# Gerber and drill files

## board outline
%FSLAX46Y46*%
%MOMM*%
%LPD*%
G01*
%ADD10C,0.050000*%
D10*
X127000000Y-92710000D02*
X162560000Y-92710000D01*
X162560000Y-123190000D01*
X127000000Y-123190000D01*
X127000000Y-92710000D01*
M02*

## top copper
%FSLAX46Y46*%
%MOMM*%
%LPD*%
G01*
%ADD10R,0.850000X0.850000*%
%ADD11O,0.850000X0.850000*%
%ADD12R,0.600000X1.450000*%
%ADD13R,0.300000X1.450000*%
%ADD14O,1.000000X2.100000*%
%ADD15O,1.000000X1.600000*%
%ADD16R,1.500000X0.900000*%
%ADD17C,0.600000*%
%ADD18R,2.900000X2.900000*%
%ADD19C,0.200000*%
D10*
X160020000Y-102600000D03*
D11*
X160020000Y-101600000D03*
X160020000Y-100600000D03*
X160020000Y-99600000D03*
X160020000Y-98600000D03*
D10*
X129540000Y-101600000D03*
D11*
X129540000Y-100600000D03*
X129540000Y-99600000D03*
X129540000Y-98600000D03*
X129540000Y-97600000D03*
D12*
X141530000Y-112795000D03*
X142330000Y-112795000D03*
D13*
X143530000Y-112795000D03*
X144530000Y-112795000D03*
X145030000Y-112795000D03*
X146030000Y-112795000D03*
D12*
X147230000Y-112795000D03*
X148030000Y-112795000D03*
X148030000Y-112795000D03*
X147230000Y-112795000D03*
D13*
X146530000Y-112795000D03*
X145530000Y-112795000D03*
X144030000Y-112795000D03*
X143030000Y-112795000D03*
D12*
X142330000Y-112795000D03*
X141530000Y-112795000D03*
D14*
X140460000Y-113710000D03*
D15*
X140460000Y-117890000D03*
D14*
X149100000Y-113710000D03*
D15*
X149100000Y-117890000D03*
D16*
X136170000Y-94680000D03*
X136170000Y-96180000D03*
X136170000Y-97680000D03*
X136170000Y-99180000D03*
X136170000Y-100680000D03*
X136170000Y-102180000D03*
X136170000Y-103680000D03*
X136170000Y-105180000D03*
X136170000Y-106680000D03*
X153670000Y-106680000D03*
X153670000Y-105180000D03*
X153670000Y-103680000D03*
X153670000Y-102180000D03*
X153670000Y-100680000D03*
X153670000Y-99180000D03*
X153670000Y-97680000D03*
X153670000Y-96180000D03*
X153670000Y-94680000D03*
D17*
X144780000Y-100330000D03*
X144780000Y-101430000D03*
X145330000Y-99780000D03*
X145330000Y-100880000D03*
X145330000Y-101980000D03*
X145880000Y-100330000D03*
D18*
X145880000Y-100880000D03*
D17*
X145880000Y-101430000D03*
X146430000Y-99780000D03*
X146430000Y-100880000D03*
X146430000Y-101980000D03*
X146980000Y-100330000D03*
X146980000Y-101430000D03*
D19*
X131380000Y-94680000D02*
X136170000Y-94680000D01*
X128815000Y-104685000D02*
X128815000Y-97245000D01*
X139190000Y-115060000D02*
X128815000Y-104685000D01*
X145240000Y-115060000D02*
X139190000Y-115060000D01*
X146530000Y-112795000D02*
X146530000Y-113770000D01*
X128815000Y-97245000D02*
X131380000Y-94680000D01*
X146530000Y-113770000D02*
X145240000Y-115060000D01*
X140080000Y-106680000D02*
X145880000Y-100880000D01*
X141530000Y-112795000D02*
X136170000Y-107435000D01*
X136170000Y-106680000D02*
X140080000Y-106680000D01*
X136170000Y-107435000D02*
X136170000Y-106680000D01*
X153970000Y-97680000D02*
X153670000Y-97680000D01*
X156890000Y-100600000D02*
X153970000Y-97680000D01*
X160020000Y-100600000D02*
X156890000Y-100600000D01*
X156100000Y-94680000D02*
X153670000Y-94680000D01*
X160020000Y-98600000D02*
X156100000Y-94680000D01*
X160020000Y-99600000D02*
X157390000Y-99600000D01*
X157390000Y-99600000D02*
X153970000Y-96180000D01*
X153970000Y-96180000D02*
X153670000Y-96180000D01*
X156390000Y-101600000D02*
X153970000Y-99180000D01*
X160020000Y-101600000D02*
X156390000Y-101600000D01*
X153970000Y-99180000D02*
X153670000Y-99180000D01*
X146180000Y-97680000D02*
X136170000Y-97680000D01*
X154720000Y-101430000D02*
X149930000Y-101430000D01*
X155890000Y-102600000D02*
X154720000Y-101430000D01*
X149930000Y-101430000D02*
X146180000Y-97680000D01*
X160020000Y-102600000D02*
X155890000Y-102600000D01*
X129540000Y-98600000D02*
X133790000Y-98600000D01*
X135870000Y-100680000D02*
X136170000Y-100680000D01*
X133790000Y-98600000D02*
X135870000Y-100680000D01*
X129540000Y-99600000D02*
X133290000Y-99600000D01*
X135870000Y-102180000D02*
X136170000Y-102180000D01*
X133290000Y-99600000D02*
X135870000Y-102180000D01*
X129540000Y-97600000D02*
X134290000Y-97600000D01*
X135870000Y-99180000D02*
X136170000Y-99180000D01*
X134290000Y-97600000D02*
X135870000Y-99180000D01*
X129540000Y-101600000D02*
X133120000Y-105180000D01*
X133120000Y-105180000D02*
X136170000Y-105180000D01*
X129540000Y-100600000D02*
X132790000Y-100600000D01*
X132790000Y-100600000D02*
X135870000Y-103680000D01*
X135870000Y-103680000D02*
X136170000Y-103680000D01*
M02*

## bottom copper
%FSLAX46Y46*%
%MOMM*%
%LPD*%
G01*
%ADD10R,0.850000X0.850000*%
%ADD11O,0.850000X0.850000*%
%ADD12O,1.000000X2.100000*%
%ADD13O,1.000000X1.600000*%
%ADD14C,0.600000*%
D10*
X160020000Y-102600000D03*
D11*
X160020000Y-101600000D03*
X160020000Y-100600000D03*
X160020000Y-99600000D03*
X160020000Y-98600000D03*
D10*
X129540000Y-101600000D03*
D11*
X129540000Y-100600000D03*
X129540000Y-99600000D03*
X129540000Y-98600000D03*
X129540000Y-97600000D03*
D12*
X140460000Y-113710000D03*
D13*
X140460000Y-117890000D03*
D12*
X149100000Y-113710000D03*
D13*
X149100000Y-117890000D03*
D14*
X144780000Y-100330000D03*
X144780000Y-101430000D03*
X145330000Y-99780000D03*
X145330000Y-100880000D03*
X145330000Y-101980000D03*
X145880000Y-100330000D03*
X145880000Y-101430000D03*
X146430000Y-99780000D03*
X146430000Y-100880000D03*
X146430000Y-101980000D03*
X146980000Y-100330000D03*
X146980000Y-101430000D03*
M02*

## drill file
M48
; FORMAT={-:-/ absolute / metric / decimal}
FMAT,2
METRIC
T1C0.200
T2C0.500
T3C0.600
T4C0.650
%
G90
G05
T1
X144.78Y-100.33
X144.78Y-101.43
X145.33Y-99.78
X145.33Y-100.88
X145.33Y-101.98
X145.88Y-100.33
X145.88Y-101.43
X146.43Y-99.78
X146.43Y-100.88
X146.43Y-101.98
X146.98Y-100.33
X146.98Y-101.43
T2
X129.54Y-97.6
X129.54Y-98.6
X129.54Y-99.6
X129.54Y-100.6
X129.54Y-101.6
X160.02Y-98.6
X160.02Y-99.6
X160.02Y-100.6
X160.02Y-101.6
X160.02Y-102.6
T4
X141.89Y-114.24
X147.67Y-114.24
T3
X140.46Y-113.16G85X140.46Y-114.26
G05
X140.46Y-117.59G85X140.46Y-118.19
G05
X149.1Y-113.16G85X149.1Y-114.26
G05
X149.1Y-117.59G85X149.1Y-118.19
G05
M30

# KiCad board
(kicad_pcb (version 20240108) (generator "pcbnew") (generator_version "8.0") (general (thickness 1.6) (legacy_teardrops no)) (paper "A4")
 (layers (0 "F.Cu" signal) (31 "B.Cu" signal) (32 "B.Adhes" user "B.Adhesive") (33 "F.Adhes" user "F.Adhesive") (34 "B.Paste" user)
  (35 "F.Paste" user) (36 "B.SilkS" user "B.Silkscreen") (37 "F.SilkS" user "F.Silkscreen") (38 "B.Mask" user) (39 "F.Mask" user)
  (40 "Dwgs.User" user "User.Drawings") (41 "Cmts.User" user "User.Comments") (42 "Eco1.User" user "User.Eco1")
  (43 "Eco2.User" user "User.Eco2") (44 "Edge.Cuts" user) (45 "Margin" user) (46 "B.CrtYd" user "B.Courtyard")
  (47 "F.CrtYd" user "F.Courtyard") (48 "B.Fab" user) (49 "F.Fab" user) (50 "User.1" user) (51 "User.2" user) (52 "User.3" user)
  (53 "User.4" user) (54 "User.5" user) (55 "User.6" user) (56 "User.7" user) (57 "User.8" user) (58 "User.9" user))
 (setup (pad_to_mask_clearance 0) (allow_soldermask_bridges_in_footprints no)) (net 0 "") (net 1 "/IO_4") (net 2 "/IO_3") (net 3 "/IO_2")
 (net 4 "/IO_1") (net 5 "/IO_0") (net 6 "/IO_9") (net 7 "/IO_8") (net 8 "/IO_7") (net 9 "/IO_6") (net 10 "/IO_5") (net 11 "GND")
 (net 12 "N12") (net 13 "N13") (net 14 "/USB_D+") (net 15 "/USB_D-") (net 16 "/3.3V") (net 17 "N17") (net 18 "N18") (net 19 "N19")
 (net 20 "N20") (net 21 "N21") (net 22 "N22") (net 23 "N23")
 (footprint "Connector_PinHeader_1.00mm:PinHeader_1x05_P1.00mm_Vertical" (layer "F.Cu") (at 160.02 102.6 180)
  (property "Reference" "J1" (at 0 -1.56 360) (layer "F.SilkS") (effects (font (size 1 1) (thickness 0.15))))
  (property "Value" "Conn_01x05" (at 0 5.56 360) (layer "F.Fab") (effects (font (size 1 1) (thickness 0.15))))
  (pad "1" thru_hole rect (at 0 0 180) (size 0.85 0.85) (drill 0.5) (layers "*.Cu" "*.Mask") (remove_unused_layers no) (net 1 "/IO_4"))
  (pad "2" thru_hole oval (at 0 1 180) (size 0.85 0.85) (drill 0.5) (layers "*.Cu" "*.Mask") (remove_unused_layers no) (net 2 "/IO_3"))
  (pad "3" thru_hole oval (at 0 2 180) (size 0.85 0.85) (drill 0.5) (layers "*.Cu" "*.Mask") (remove_unused_layers no) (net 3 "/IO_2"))
  (pad "4" thru_hole oval (at 0 3 180) (size 0.85 0.85) (drill 0.5) (layers "*.Cu" "*.Mask") (remove_unused_layers no) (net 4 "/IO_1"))
  (pad "5" thru_hole oval (at 0 4 180) (size 0.85 0.85) (drill 0.5) (layers "*.Cu" "*.Mask") (remove_unused_layers no) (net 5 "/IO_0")))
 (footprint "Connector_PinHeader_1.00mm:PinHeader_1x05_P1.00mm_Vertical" (layer "F.Cu") (at 129.54 101.6 180)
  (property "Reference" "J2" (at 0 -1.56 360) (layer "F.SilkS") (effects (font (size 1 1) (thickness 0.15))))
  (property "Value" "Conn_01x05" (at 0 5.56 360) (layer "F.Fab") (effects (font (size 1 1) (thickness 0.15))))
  (pad "1" thru_hole rect (at 0 0 180) (size 0.85 0.85) (drill 0.5) (layers "*.Cu" "*.Mask") (remove_unused_layers no) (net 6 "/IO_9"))
  (pad "2" thru_hole oval (at 0 1 180) (size 0.85 0.85) (drill 0.5) (layers "*.Cu" "*.Mask") (remove_unused_layers no) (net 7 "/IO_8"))
  (pad "3" thru_hole oval (at 0 2 180) (size 0.85 0.85) (drill 0.5) (layers "*.Cu" "*.Mask") (remove_unused_layers no) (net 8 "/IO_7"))
  (pad "4" thru_hole oval (at 0 3 180) (size 0.85 0.85) (drill 0.5) (layers "*.Cu" "*.Mask") (remove_unused_layers no) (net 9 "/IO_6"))
  (pad "5" thru_hole oval (at 0 4 180) (size 0.85 0.85) (drill 0.5) (layers "*.Cu" "*.Mask") (remove_unused_layers no) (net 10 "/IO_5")))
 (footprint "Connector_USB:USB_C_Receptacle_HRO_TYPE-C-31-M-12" (layer "F.Cu") (at 144.78 116.84)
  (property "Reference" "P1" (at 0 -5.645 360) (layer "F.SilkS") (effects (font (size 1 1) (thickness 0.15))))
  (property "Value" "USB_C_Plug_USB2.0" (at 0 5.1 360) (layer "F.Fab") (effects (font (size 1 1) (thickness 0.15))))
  (pad "" np_thru_hole circle (at -2.89 -2.6) (size 0.65 0.65) (drill 0.65) (layers "*.Cu" "*.Mask"))
  (pad "" np_thru_hole circle (at 2.89 -2.6) (size 0.65 0.65) (drill 0.65) (layers "*.Cu" "*.Mask"))
  (pad "A1" smd rect (at -3.25 -4.045) (size 0.6 1.45) (layers "F.Cu" "F.Paste" "F.Mask") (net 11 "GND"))
  (pad "A4" smd rect (at -2.45 -4.045) (size 0.6 1.45) (layers "F.Cu" "F.Paste" "F.Mask") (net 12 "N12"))
  (pad "A5" smd rect (at -1.25 -4.045) (size 0.3 1.45) (layers "F.Cu" "F.Paste" "F.Mask") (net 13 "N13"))
  (pad "A6" smd rect (at -0.25 -4.045) (size 0.3 1.45) (layers "F.Cu" "F.Paste" "F.Mask") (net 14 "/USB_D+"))
  (pad "A7" smd rect (at 0.25 -4.045) (size 0.3 1.45) (layers "F.Cu" "F.Paste" "F.Mask") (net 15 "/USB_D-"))
  (pad "A8" smd rect (at 1.25 -4.045) (size 0.3 1.45) (layers "F.Cu" "F.Paste" "F.Mask"))
  (pad "A9" smd rect (at 2.45 -4.045) (size 0.6 1.45) (layers "F.Cu" "F.Paste" "F.Mask") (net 12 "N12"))
  (pad "A12" smd rect (at 3.25 -4.045) (size 0.6 1.45) (layers "F.Cu" "F.Paste" "F.Mask") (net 11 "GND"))
  (pad "B1" smd rect (at 3.25 -4.045) (size 0.6 1.45) (layers "F.Cu" "F.Paste" "F.Mask") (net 11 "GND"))
  (pad "B4" smd rect (at 2.45 -4.045) (size 0.6 1.45) (layers "F.Cu" "F.Paste" "F.Mask") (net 12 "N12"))
  (pad "B5" smd rect (at 1.75 -4.045) (size 0.3 1.45) (layers "F.Cu" "F.Paste" "F.Mask") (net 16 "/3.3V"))
  (pad "B6" smd rect (at 0.75 -4.045) (size 0.3 1.45) (layers "F.Cu" "F.Paste" "F.Mask"))
  (pad "B7" smd rect (at -0.75 -4.045) (size 0.3 1.45) (layers "F.Cu" "F.Paste" "F.Mask"))
  (pad "B8" smd rect (at -1.75 -4.045) (size 0.3 1.45) (layers "F.Cu" "F.Paste" "F.Mask"))
  (pad "B9" smd rect (at -2.45 -4.045) (size 0.6 1.45) (layers "F.Cu" "F.Paste" "F.Mask") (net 12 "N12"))
  (pad "B12" smd rect (at -3.25 -4.045) (size 0.6 1.45) (layers "F.Cu" "F.Paste" "F.Mask") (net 11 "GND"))
  (pad "S1" thru_hole oval (at -4.32 -3.13) (size 1 2.1) (drill oval 0.6 1.7) (layers "*.Cu" "*.Mask") (remove_unused_layers no)
   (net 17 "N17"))
  (pad "S1" thru_hole oval (at -4.32 1.05) (size 1 1.6) (drill oval 0.6 1.2) (layers "*.Cu" "*.Mask") (remove_unused_layers no)
   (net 17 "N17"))
  (pad "S1" thru_hole oval (at 4.32 -3.13) (size 1 2.1) (drill oval 0.6 1.7) (layers "*.Cu" "*.Mask") (remove_unused_layers no)
   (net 17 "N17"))
  (pad "S1" thru_hole oval (at 4.32 1.05) (size 1 1.6) (drill oval 0.6 1.2) (layers "*.Cu" "*.Mask") (remove_unused_layers no)
   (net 17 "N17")))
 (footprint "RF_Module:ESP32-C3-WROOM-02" (layer "F.Cu") (at 144.92 100.68)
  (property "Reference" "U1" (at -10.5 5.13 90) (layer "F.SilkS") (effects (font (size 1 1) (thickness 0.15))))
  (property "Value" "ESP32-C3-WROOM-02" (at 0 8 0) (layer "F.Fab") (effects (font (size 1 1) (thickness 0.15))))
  (pad "" smd rect (at -0.14 -0.9) (size 0.7 0.7) (layers "F.Paste"))
  (pad "" smd rect (at -0.14 0.2) (size 0.7 0.7) (layers "F.Paste"))
  (pad "" smd rect (at -0.14 1.3) (size 0.7 0.7) (layers "F.Paste"))
  (pad "" smd rect (at 0.96 -0.9) (size 0.7 0.7) (layers "F.Paste"))
  (pad "" smd rect (at 0.96 0.2) (size 0.7 0.7) (layers "F.Paste"))
  (pad "" smd rect (at 0.96 1.3) (size 0.7 0.7) (layers "F.Paste"))
  (pad "" smd rect (at 2.06 -0.9) (size 0.7 0.7) (layers "F.Paste"))
  (pad "" smd rect (at 2.06 0.2) (size 0.7 0.7) (layers "F.Paste"))
  (pad "" smd rect (at 2.06 1.3) (size 0.7 0.7) (layers "F.Paste"))
  (pad "1" smd rect (at -8.75 -6) (size 1.5 0.9) (layers "F.Cu" "F.Paste" "F.Mask") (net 16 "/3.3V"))
  (pad "2" smd rect (at -8.75 -4.5) (size 1.5 0.9) (layers "F.Cu" "F.Paste" "F.Mask") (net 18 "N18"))
  (pad "3" smd rect (at -8.75 -3) (size 1.5 0.9) (layers "F.Cu" "F.Paste" "F.Mask") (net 1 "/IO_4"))
  (pad "4" smd rect (at -8.75 -1.5) (size 1.5 0.9) (layers "F.Cu" "F.Paste" "F.Mask") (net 10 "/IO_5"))
  (pad "5" smd rect (at -8.75 0) (size 1.5 0.9) (layers "F.Cu" "F.Paste" "F.Mask") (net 9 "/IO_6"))
  (pad "6" smd rect (at -8.75 1.5) (size 1.5 0.9) (layers "F.Cu" "F.Paste" "F.Mask") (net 8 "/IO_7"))
  (pad "7" smd rect (at -8.75 3) (size 1.5 0.9) (layers "F.Cu" "F.Paste" "F.Mask") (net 7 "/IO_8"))
  (pad "8" smd rect (at -8.75 4.5) (size 1.5 0.9) (layers "F.Cu" "F.Paste" "F.Mask") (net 6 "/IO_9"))
  (pad "9" smd rect (at -8.75 6) (size 1.5 0.9) (layers "F.Cu" "F.Paste" "F.Mask") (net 11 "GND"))
  (pad "10" smd rect (at 8.75 6) (size 1.5 0.9) (layers "F.Cu" "F.Paste" "F.Mask") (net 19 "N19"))
  (pad "11" smd rect (at 8.75 4.5) (size 1.5 0.9) (layers "F.Cu" "F.Paste" "F.Mask") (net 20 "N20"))
  (pad "12" smd rect (at 8.75 3) (size 1.5 0.9) (layers "F.Cu" "F.Paste" "F.Mask") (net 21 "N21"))
  (pad "13" smd rect (at 8.75 1.5) (size 1.5 0.9) (layers "F.Cu" "F.Paste" "F.Mask") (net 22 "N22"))
  (pad "14" smd rect (at 8.75 0) (size 1.5 0.9) (layers "F.Cu" "F.Paste" "F.Mask") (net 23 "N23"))
  (pad "15" smd rect (at 8.75 -1.5) (size 1.5 0.9) (layers "F.Cu" "F.Paste" "F.Mask") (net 2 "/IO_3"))
  (pad "16" smd rect (at 8.75 -3) (size 1.5 0.9) (layers "F.Cu" "F.Paste" "F.Mask") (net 3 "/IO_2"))
  (pad "17" smd rect (at 8.75 -4.5) (size 1.5 0.9) (layers "F.Cu" "F.Paste" "F.Mask") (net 4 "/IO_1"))
  (pad "18" smd rect (at 8.75 -6) (size 1.5 0.9) (layers "F.Cu" "F.Paste" "F.Mask") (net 5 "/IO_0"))
  (pad "19" thru_hole circle (at -0.14 -0.35) (size 0.6 0.6) (drill 0.2) (layers "*.Cu" "F.Mask") (remove_unused_layers no) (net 11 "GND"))
  (pad "19" thru_hole circle (at -0.14 0.75) (size 0.6 0.6) (drill 0.2) (layers "*.Cu" "F.Mask") (remove_unused_layers no) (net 11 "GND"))
  (pad "19" thru_hole circle (at 0.41 -0.9) (size 0.6 0.6) (drill 0.2) (layers "*.Cu" "F.Mask") (remove_unused_layers no) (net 11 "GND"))
  (pad "19" thru_hole circle (at 0.41 0.2) (size 0.6 0.6) (drill 0.2) (layers "*.Cu" "F.Mask") (remove_unused_layers no) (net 11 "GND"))
  (pad "19" thru_hole circle (at 0.41 1.3) (size 0.6 0.6) (drill 0.2) (layers "*.Cu" "F.Mask") (remove_unused_layers no) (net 11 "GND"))
  (pad "19" thru_hole circle (at 0.96 -0.35) (size 0.6 0.6) (drill 0.2) (layers "*.Cu" "F.Mask") (remove_unused_layers no) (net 11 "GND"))
  (pad "19" smd rect (at 0.96 0.2) (size 2.9 2.9) (layers "F.Cu" "F.Mask") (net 11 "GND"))
  (pad "19" thru_hole circle (at 0.96 0.75) (size 0.6 0.6) (drill 0.2) (layers "*.Cu" "F.Mask") (remove_unused_layers no) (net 11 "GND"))
  (pad "19" thru_hole circle (at 1.51 -0.9) (size 0.6 0.6) (drill 0.2) (layers "*.Cu" "F.Mask") (remove_unused_layers no) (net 11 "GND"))
  (pad "19" thru_hole circle (at 1.51 0.2) (size 0.6 0.6) (drill 0.2) (layers "*.Cu" "F.Mask") (remove_unused_layers no) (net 11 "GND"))
  (pad "19" thru_hole circle (at 1.51 1.3) (size 0.6 0.6) (drill 0.2) (layers "*.Cu" "F.Mask") (remove_unused_layers no) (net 11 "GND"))
  (pad "19" thru_hole circle (at 2.06 -0.35) (size 0.6 0.6) (drill 0.2) (layers "*.Cu" "F.Mask") (remove_unused_layers no) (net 11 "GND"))
  (pad "19" thru_hole circle (at 2.06 0.75) (size 0.6 0.6) (drill 0.2) (layers "*.Cu" "F.Mask") (remove_unused_layers no) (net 11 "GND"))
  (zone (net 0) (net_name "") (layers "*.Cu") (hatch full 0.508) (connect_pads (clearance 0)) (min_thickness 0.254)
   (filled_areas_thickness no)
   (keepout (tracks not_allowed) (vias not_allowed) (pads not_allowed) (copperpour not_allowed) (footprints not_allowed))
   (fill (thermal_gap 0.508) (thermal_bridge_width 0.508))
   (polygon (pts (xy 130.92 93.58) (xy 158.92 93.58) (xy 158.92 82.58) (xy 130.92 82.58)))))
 (gr_rect (start 127 92.71) (end 162.56 123.19) (stroke (width 0.05) (type default)) (fill none) (layer "Edge.Cuts"))
 (segment (start 131.38 94.68) (end 136.17 94.68) (width 0.2) (layer "F.Cu") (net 16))
 (segment (start 128.815 104.685) (end 128.815 97.245) (width 0.2) (layer "F.Cu") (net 16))
 (segment (start 139.19 115.06) (end 128.815 104.685) (width 0.2) (layer "F.Cu") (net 16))
 (segment (start 145.24 115.06) (end 139.19 115.06) (width 0.2) (layer "F.Cu") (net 16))
 (segment (start 146.53 112.795) (end 146.53 113.77) (width 0.2) (layer "F.Cu") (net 16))
 (segment (start 128.815 97.245) (end 131.38 94.68) (width 0.2) (layer "F.Cu") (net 16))
 (segment (start 146.53 113.77) (end 145.24 115.06) (width 0.2) (layer "F.Cu") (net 16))
 (segment (start 140.08 106.68) (end 145.88 100.88) (width 0.2) (layer "F.Cu") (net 11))
 (segment (start 141.53 112.795) (end 136.17 107.435) (width 0.2) (layer "F.Cu") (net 11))
 (segment (start 136.17 106.68) (end 140.08 106.68) (width 0.2) (layer "F.Cu") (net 11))
 (segment (start 136.17 107.435) (end 136.17 106.68) (width 0.2) (layer "F.Cu") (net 11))
 (segment (start 153.97 97.68) (end 153.67 97.68) (width 0.2) (layer "F.Cu") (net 3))
 (segment (start 156.89 100.6) (end 153.97 97.68) (width 0.2) (layer "F.Cu") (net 3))
 (segment (start 160.02 100.6) (end 156.89 100.6) (width 0.2) (layer "F.Cu") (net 3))
 (segment (start 156.1 94.68) (end 153.67 94.68) (width 0.2) (layer "F.Cu") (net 5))
 (segment (start 160.02 98.6) (end 156.1 94.68) (width 0.2) (layer "F.Cu") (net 5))
 (segment (start 160.02 99.6) (end 157.39 99.6) (width 0.2) (layer "F.Cu") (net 4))
 (segment (start 157.39 99.6) (end 153.97 96.18) (width 0.2) (layer "F.Cu") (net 4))
 (segment (start 153.97 96.18) (end 153.67 96.18) (width 0.2) (layer "F.Cu") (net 4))
 (segment (start 156.39 101.6) (end 153.97 99.18) (width 0.2) (layer "F.Cu") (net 2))
 (segment (start 160.02 101.6) (end 156.39 101.6) (width 0.2) (layer "F.Cu") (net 2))
 (segment (start 153.97 99.18) (end 153.67 99.18) (width 0.2) (layer "F.Cu") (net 2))
 (segment (start 146.18 97.68) (end 136.17 97.68) (width 0.2) (layer "F.Cu") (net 1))
 (segment (start 154.72 101.43) (end 149.93 101.43) (width 0.2) (layer "F.Cu") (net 1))
 (segment (start 155.89 102.6) (end 154.72 101.43) (width 0.2) (layer "F.Cu") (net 1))
 (segment (start 149.93 101.43) (end 146.18 97.68) (width 0.2) (layer "F.Cu") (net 1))
 (segment (start 160.02 102.6) (end 155.89 102.6) (width 0.2) (layer "F.Cu") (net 1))
 (segment (start 129.54 98.6) (end 133.79 98.6) (width 0.2) (layer "F.Cu") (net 9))
 (segment (start 135.87 100.68) (end 136.17 100.68) (width 0.2) (layer "F.Cu") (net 9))
 (segment (start 133.79 98.6) (end 135.87 100.68) (width 0.2) (layer "F.Cu") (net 9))
 (segment (start 129.54 99.6) (end 133.29 99.6) (width 0.2) (layer "F.Cu") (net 8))
 (segment (start 135.87 102.18) (end 136.17 102.18) (width 0.2) (layer "F.Cu") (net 8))
 (segment (start 133.29 99.6) (end 135.87 102.18) (width 0.2) (layer "F.Cu") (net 8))
 (segment (start 129.54 97.6) (end 134.29 97.6) (width 0.2) (layer "F.Cu") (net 10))
 (segment (start 135.87 99.18) (end 136.17 99.18) (width 0.2) (layer "F.Cu") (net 10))
 (segment (start 134.29 97.6) (end 135.87 99.18) (width 0.2) (layer "F.Cu") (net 10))
 (segment (start 129.54 101.6) (end 133.12 105.18) (width 0.2) (layer "F.Cu") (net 6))
 (segment (start 133.12 105.18) (end 136.17 105.18) (width 0.2) (layer "F.Cu") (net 6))
 (segment (start 129.54 100.6) (end 132.79 100.6) (width 0.2) (layer "F.Cu") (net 7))
 (segment (start 132.79 100.6) (end 135.87 103.68) (width 0.2) (layer "F.Cu") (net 7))
 (segment (start 135.87 103.68) (end 136.17 103.68) (width 0.2) (layer "F.Cu") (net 7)))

